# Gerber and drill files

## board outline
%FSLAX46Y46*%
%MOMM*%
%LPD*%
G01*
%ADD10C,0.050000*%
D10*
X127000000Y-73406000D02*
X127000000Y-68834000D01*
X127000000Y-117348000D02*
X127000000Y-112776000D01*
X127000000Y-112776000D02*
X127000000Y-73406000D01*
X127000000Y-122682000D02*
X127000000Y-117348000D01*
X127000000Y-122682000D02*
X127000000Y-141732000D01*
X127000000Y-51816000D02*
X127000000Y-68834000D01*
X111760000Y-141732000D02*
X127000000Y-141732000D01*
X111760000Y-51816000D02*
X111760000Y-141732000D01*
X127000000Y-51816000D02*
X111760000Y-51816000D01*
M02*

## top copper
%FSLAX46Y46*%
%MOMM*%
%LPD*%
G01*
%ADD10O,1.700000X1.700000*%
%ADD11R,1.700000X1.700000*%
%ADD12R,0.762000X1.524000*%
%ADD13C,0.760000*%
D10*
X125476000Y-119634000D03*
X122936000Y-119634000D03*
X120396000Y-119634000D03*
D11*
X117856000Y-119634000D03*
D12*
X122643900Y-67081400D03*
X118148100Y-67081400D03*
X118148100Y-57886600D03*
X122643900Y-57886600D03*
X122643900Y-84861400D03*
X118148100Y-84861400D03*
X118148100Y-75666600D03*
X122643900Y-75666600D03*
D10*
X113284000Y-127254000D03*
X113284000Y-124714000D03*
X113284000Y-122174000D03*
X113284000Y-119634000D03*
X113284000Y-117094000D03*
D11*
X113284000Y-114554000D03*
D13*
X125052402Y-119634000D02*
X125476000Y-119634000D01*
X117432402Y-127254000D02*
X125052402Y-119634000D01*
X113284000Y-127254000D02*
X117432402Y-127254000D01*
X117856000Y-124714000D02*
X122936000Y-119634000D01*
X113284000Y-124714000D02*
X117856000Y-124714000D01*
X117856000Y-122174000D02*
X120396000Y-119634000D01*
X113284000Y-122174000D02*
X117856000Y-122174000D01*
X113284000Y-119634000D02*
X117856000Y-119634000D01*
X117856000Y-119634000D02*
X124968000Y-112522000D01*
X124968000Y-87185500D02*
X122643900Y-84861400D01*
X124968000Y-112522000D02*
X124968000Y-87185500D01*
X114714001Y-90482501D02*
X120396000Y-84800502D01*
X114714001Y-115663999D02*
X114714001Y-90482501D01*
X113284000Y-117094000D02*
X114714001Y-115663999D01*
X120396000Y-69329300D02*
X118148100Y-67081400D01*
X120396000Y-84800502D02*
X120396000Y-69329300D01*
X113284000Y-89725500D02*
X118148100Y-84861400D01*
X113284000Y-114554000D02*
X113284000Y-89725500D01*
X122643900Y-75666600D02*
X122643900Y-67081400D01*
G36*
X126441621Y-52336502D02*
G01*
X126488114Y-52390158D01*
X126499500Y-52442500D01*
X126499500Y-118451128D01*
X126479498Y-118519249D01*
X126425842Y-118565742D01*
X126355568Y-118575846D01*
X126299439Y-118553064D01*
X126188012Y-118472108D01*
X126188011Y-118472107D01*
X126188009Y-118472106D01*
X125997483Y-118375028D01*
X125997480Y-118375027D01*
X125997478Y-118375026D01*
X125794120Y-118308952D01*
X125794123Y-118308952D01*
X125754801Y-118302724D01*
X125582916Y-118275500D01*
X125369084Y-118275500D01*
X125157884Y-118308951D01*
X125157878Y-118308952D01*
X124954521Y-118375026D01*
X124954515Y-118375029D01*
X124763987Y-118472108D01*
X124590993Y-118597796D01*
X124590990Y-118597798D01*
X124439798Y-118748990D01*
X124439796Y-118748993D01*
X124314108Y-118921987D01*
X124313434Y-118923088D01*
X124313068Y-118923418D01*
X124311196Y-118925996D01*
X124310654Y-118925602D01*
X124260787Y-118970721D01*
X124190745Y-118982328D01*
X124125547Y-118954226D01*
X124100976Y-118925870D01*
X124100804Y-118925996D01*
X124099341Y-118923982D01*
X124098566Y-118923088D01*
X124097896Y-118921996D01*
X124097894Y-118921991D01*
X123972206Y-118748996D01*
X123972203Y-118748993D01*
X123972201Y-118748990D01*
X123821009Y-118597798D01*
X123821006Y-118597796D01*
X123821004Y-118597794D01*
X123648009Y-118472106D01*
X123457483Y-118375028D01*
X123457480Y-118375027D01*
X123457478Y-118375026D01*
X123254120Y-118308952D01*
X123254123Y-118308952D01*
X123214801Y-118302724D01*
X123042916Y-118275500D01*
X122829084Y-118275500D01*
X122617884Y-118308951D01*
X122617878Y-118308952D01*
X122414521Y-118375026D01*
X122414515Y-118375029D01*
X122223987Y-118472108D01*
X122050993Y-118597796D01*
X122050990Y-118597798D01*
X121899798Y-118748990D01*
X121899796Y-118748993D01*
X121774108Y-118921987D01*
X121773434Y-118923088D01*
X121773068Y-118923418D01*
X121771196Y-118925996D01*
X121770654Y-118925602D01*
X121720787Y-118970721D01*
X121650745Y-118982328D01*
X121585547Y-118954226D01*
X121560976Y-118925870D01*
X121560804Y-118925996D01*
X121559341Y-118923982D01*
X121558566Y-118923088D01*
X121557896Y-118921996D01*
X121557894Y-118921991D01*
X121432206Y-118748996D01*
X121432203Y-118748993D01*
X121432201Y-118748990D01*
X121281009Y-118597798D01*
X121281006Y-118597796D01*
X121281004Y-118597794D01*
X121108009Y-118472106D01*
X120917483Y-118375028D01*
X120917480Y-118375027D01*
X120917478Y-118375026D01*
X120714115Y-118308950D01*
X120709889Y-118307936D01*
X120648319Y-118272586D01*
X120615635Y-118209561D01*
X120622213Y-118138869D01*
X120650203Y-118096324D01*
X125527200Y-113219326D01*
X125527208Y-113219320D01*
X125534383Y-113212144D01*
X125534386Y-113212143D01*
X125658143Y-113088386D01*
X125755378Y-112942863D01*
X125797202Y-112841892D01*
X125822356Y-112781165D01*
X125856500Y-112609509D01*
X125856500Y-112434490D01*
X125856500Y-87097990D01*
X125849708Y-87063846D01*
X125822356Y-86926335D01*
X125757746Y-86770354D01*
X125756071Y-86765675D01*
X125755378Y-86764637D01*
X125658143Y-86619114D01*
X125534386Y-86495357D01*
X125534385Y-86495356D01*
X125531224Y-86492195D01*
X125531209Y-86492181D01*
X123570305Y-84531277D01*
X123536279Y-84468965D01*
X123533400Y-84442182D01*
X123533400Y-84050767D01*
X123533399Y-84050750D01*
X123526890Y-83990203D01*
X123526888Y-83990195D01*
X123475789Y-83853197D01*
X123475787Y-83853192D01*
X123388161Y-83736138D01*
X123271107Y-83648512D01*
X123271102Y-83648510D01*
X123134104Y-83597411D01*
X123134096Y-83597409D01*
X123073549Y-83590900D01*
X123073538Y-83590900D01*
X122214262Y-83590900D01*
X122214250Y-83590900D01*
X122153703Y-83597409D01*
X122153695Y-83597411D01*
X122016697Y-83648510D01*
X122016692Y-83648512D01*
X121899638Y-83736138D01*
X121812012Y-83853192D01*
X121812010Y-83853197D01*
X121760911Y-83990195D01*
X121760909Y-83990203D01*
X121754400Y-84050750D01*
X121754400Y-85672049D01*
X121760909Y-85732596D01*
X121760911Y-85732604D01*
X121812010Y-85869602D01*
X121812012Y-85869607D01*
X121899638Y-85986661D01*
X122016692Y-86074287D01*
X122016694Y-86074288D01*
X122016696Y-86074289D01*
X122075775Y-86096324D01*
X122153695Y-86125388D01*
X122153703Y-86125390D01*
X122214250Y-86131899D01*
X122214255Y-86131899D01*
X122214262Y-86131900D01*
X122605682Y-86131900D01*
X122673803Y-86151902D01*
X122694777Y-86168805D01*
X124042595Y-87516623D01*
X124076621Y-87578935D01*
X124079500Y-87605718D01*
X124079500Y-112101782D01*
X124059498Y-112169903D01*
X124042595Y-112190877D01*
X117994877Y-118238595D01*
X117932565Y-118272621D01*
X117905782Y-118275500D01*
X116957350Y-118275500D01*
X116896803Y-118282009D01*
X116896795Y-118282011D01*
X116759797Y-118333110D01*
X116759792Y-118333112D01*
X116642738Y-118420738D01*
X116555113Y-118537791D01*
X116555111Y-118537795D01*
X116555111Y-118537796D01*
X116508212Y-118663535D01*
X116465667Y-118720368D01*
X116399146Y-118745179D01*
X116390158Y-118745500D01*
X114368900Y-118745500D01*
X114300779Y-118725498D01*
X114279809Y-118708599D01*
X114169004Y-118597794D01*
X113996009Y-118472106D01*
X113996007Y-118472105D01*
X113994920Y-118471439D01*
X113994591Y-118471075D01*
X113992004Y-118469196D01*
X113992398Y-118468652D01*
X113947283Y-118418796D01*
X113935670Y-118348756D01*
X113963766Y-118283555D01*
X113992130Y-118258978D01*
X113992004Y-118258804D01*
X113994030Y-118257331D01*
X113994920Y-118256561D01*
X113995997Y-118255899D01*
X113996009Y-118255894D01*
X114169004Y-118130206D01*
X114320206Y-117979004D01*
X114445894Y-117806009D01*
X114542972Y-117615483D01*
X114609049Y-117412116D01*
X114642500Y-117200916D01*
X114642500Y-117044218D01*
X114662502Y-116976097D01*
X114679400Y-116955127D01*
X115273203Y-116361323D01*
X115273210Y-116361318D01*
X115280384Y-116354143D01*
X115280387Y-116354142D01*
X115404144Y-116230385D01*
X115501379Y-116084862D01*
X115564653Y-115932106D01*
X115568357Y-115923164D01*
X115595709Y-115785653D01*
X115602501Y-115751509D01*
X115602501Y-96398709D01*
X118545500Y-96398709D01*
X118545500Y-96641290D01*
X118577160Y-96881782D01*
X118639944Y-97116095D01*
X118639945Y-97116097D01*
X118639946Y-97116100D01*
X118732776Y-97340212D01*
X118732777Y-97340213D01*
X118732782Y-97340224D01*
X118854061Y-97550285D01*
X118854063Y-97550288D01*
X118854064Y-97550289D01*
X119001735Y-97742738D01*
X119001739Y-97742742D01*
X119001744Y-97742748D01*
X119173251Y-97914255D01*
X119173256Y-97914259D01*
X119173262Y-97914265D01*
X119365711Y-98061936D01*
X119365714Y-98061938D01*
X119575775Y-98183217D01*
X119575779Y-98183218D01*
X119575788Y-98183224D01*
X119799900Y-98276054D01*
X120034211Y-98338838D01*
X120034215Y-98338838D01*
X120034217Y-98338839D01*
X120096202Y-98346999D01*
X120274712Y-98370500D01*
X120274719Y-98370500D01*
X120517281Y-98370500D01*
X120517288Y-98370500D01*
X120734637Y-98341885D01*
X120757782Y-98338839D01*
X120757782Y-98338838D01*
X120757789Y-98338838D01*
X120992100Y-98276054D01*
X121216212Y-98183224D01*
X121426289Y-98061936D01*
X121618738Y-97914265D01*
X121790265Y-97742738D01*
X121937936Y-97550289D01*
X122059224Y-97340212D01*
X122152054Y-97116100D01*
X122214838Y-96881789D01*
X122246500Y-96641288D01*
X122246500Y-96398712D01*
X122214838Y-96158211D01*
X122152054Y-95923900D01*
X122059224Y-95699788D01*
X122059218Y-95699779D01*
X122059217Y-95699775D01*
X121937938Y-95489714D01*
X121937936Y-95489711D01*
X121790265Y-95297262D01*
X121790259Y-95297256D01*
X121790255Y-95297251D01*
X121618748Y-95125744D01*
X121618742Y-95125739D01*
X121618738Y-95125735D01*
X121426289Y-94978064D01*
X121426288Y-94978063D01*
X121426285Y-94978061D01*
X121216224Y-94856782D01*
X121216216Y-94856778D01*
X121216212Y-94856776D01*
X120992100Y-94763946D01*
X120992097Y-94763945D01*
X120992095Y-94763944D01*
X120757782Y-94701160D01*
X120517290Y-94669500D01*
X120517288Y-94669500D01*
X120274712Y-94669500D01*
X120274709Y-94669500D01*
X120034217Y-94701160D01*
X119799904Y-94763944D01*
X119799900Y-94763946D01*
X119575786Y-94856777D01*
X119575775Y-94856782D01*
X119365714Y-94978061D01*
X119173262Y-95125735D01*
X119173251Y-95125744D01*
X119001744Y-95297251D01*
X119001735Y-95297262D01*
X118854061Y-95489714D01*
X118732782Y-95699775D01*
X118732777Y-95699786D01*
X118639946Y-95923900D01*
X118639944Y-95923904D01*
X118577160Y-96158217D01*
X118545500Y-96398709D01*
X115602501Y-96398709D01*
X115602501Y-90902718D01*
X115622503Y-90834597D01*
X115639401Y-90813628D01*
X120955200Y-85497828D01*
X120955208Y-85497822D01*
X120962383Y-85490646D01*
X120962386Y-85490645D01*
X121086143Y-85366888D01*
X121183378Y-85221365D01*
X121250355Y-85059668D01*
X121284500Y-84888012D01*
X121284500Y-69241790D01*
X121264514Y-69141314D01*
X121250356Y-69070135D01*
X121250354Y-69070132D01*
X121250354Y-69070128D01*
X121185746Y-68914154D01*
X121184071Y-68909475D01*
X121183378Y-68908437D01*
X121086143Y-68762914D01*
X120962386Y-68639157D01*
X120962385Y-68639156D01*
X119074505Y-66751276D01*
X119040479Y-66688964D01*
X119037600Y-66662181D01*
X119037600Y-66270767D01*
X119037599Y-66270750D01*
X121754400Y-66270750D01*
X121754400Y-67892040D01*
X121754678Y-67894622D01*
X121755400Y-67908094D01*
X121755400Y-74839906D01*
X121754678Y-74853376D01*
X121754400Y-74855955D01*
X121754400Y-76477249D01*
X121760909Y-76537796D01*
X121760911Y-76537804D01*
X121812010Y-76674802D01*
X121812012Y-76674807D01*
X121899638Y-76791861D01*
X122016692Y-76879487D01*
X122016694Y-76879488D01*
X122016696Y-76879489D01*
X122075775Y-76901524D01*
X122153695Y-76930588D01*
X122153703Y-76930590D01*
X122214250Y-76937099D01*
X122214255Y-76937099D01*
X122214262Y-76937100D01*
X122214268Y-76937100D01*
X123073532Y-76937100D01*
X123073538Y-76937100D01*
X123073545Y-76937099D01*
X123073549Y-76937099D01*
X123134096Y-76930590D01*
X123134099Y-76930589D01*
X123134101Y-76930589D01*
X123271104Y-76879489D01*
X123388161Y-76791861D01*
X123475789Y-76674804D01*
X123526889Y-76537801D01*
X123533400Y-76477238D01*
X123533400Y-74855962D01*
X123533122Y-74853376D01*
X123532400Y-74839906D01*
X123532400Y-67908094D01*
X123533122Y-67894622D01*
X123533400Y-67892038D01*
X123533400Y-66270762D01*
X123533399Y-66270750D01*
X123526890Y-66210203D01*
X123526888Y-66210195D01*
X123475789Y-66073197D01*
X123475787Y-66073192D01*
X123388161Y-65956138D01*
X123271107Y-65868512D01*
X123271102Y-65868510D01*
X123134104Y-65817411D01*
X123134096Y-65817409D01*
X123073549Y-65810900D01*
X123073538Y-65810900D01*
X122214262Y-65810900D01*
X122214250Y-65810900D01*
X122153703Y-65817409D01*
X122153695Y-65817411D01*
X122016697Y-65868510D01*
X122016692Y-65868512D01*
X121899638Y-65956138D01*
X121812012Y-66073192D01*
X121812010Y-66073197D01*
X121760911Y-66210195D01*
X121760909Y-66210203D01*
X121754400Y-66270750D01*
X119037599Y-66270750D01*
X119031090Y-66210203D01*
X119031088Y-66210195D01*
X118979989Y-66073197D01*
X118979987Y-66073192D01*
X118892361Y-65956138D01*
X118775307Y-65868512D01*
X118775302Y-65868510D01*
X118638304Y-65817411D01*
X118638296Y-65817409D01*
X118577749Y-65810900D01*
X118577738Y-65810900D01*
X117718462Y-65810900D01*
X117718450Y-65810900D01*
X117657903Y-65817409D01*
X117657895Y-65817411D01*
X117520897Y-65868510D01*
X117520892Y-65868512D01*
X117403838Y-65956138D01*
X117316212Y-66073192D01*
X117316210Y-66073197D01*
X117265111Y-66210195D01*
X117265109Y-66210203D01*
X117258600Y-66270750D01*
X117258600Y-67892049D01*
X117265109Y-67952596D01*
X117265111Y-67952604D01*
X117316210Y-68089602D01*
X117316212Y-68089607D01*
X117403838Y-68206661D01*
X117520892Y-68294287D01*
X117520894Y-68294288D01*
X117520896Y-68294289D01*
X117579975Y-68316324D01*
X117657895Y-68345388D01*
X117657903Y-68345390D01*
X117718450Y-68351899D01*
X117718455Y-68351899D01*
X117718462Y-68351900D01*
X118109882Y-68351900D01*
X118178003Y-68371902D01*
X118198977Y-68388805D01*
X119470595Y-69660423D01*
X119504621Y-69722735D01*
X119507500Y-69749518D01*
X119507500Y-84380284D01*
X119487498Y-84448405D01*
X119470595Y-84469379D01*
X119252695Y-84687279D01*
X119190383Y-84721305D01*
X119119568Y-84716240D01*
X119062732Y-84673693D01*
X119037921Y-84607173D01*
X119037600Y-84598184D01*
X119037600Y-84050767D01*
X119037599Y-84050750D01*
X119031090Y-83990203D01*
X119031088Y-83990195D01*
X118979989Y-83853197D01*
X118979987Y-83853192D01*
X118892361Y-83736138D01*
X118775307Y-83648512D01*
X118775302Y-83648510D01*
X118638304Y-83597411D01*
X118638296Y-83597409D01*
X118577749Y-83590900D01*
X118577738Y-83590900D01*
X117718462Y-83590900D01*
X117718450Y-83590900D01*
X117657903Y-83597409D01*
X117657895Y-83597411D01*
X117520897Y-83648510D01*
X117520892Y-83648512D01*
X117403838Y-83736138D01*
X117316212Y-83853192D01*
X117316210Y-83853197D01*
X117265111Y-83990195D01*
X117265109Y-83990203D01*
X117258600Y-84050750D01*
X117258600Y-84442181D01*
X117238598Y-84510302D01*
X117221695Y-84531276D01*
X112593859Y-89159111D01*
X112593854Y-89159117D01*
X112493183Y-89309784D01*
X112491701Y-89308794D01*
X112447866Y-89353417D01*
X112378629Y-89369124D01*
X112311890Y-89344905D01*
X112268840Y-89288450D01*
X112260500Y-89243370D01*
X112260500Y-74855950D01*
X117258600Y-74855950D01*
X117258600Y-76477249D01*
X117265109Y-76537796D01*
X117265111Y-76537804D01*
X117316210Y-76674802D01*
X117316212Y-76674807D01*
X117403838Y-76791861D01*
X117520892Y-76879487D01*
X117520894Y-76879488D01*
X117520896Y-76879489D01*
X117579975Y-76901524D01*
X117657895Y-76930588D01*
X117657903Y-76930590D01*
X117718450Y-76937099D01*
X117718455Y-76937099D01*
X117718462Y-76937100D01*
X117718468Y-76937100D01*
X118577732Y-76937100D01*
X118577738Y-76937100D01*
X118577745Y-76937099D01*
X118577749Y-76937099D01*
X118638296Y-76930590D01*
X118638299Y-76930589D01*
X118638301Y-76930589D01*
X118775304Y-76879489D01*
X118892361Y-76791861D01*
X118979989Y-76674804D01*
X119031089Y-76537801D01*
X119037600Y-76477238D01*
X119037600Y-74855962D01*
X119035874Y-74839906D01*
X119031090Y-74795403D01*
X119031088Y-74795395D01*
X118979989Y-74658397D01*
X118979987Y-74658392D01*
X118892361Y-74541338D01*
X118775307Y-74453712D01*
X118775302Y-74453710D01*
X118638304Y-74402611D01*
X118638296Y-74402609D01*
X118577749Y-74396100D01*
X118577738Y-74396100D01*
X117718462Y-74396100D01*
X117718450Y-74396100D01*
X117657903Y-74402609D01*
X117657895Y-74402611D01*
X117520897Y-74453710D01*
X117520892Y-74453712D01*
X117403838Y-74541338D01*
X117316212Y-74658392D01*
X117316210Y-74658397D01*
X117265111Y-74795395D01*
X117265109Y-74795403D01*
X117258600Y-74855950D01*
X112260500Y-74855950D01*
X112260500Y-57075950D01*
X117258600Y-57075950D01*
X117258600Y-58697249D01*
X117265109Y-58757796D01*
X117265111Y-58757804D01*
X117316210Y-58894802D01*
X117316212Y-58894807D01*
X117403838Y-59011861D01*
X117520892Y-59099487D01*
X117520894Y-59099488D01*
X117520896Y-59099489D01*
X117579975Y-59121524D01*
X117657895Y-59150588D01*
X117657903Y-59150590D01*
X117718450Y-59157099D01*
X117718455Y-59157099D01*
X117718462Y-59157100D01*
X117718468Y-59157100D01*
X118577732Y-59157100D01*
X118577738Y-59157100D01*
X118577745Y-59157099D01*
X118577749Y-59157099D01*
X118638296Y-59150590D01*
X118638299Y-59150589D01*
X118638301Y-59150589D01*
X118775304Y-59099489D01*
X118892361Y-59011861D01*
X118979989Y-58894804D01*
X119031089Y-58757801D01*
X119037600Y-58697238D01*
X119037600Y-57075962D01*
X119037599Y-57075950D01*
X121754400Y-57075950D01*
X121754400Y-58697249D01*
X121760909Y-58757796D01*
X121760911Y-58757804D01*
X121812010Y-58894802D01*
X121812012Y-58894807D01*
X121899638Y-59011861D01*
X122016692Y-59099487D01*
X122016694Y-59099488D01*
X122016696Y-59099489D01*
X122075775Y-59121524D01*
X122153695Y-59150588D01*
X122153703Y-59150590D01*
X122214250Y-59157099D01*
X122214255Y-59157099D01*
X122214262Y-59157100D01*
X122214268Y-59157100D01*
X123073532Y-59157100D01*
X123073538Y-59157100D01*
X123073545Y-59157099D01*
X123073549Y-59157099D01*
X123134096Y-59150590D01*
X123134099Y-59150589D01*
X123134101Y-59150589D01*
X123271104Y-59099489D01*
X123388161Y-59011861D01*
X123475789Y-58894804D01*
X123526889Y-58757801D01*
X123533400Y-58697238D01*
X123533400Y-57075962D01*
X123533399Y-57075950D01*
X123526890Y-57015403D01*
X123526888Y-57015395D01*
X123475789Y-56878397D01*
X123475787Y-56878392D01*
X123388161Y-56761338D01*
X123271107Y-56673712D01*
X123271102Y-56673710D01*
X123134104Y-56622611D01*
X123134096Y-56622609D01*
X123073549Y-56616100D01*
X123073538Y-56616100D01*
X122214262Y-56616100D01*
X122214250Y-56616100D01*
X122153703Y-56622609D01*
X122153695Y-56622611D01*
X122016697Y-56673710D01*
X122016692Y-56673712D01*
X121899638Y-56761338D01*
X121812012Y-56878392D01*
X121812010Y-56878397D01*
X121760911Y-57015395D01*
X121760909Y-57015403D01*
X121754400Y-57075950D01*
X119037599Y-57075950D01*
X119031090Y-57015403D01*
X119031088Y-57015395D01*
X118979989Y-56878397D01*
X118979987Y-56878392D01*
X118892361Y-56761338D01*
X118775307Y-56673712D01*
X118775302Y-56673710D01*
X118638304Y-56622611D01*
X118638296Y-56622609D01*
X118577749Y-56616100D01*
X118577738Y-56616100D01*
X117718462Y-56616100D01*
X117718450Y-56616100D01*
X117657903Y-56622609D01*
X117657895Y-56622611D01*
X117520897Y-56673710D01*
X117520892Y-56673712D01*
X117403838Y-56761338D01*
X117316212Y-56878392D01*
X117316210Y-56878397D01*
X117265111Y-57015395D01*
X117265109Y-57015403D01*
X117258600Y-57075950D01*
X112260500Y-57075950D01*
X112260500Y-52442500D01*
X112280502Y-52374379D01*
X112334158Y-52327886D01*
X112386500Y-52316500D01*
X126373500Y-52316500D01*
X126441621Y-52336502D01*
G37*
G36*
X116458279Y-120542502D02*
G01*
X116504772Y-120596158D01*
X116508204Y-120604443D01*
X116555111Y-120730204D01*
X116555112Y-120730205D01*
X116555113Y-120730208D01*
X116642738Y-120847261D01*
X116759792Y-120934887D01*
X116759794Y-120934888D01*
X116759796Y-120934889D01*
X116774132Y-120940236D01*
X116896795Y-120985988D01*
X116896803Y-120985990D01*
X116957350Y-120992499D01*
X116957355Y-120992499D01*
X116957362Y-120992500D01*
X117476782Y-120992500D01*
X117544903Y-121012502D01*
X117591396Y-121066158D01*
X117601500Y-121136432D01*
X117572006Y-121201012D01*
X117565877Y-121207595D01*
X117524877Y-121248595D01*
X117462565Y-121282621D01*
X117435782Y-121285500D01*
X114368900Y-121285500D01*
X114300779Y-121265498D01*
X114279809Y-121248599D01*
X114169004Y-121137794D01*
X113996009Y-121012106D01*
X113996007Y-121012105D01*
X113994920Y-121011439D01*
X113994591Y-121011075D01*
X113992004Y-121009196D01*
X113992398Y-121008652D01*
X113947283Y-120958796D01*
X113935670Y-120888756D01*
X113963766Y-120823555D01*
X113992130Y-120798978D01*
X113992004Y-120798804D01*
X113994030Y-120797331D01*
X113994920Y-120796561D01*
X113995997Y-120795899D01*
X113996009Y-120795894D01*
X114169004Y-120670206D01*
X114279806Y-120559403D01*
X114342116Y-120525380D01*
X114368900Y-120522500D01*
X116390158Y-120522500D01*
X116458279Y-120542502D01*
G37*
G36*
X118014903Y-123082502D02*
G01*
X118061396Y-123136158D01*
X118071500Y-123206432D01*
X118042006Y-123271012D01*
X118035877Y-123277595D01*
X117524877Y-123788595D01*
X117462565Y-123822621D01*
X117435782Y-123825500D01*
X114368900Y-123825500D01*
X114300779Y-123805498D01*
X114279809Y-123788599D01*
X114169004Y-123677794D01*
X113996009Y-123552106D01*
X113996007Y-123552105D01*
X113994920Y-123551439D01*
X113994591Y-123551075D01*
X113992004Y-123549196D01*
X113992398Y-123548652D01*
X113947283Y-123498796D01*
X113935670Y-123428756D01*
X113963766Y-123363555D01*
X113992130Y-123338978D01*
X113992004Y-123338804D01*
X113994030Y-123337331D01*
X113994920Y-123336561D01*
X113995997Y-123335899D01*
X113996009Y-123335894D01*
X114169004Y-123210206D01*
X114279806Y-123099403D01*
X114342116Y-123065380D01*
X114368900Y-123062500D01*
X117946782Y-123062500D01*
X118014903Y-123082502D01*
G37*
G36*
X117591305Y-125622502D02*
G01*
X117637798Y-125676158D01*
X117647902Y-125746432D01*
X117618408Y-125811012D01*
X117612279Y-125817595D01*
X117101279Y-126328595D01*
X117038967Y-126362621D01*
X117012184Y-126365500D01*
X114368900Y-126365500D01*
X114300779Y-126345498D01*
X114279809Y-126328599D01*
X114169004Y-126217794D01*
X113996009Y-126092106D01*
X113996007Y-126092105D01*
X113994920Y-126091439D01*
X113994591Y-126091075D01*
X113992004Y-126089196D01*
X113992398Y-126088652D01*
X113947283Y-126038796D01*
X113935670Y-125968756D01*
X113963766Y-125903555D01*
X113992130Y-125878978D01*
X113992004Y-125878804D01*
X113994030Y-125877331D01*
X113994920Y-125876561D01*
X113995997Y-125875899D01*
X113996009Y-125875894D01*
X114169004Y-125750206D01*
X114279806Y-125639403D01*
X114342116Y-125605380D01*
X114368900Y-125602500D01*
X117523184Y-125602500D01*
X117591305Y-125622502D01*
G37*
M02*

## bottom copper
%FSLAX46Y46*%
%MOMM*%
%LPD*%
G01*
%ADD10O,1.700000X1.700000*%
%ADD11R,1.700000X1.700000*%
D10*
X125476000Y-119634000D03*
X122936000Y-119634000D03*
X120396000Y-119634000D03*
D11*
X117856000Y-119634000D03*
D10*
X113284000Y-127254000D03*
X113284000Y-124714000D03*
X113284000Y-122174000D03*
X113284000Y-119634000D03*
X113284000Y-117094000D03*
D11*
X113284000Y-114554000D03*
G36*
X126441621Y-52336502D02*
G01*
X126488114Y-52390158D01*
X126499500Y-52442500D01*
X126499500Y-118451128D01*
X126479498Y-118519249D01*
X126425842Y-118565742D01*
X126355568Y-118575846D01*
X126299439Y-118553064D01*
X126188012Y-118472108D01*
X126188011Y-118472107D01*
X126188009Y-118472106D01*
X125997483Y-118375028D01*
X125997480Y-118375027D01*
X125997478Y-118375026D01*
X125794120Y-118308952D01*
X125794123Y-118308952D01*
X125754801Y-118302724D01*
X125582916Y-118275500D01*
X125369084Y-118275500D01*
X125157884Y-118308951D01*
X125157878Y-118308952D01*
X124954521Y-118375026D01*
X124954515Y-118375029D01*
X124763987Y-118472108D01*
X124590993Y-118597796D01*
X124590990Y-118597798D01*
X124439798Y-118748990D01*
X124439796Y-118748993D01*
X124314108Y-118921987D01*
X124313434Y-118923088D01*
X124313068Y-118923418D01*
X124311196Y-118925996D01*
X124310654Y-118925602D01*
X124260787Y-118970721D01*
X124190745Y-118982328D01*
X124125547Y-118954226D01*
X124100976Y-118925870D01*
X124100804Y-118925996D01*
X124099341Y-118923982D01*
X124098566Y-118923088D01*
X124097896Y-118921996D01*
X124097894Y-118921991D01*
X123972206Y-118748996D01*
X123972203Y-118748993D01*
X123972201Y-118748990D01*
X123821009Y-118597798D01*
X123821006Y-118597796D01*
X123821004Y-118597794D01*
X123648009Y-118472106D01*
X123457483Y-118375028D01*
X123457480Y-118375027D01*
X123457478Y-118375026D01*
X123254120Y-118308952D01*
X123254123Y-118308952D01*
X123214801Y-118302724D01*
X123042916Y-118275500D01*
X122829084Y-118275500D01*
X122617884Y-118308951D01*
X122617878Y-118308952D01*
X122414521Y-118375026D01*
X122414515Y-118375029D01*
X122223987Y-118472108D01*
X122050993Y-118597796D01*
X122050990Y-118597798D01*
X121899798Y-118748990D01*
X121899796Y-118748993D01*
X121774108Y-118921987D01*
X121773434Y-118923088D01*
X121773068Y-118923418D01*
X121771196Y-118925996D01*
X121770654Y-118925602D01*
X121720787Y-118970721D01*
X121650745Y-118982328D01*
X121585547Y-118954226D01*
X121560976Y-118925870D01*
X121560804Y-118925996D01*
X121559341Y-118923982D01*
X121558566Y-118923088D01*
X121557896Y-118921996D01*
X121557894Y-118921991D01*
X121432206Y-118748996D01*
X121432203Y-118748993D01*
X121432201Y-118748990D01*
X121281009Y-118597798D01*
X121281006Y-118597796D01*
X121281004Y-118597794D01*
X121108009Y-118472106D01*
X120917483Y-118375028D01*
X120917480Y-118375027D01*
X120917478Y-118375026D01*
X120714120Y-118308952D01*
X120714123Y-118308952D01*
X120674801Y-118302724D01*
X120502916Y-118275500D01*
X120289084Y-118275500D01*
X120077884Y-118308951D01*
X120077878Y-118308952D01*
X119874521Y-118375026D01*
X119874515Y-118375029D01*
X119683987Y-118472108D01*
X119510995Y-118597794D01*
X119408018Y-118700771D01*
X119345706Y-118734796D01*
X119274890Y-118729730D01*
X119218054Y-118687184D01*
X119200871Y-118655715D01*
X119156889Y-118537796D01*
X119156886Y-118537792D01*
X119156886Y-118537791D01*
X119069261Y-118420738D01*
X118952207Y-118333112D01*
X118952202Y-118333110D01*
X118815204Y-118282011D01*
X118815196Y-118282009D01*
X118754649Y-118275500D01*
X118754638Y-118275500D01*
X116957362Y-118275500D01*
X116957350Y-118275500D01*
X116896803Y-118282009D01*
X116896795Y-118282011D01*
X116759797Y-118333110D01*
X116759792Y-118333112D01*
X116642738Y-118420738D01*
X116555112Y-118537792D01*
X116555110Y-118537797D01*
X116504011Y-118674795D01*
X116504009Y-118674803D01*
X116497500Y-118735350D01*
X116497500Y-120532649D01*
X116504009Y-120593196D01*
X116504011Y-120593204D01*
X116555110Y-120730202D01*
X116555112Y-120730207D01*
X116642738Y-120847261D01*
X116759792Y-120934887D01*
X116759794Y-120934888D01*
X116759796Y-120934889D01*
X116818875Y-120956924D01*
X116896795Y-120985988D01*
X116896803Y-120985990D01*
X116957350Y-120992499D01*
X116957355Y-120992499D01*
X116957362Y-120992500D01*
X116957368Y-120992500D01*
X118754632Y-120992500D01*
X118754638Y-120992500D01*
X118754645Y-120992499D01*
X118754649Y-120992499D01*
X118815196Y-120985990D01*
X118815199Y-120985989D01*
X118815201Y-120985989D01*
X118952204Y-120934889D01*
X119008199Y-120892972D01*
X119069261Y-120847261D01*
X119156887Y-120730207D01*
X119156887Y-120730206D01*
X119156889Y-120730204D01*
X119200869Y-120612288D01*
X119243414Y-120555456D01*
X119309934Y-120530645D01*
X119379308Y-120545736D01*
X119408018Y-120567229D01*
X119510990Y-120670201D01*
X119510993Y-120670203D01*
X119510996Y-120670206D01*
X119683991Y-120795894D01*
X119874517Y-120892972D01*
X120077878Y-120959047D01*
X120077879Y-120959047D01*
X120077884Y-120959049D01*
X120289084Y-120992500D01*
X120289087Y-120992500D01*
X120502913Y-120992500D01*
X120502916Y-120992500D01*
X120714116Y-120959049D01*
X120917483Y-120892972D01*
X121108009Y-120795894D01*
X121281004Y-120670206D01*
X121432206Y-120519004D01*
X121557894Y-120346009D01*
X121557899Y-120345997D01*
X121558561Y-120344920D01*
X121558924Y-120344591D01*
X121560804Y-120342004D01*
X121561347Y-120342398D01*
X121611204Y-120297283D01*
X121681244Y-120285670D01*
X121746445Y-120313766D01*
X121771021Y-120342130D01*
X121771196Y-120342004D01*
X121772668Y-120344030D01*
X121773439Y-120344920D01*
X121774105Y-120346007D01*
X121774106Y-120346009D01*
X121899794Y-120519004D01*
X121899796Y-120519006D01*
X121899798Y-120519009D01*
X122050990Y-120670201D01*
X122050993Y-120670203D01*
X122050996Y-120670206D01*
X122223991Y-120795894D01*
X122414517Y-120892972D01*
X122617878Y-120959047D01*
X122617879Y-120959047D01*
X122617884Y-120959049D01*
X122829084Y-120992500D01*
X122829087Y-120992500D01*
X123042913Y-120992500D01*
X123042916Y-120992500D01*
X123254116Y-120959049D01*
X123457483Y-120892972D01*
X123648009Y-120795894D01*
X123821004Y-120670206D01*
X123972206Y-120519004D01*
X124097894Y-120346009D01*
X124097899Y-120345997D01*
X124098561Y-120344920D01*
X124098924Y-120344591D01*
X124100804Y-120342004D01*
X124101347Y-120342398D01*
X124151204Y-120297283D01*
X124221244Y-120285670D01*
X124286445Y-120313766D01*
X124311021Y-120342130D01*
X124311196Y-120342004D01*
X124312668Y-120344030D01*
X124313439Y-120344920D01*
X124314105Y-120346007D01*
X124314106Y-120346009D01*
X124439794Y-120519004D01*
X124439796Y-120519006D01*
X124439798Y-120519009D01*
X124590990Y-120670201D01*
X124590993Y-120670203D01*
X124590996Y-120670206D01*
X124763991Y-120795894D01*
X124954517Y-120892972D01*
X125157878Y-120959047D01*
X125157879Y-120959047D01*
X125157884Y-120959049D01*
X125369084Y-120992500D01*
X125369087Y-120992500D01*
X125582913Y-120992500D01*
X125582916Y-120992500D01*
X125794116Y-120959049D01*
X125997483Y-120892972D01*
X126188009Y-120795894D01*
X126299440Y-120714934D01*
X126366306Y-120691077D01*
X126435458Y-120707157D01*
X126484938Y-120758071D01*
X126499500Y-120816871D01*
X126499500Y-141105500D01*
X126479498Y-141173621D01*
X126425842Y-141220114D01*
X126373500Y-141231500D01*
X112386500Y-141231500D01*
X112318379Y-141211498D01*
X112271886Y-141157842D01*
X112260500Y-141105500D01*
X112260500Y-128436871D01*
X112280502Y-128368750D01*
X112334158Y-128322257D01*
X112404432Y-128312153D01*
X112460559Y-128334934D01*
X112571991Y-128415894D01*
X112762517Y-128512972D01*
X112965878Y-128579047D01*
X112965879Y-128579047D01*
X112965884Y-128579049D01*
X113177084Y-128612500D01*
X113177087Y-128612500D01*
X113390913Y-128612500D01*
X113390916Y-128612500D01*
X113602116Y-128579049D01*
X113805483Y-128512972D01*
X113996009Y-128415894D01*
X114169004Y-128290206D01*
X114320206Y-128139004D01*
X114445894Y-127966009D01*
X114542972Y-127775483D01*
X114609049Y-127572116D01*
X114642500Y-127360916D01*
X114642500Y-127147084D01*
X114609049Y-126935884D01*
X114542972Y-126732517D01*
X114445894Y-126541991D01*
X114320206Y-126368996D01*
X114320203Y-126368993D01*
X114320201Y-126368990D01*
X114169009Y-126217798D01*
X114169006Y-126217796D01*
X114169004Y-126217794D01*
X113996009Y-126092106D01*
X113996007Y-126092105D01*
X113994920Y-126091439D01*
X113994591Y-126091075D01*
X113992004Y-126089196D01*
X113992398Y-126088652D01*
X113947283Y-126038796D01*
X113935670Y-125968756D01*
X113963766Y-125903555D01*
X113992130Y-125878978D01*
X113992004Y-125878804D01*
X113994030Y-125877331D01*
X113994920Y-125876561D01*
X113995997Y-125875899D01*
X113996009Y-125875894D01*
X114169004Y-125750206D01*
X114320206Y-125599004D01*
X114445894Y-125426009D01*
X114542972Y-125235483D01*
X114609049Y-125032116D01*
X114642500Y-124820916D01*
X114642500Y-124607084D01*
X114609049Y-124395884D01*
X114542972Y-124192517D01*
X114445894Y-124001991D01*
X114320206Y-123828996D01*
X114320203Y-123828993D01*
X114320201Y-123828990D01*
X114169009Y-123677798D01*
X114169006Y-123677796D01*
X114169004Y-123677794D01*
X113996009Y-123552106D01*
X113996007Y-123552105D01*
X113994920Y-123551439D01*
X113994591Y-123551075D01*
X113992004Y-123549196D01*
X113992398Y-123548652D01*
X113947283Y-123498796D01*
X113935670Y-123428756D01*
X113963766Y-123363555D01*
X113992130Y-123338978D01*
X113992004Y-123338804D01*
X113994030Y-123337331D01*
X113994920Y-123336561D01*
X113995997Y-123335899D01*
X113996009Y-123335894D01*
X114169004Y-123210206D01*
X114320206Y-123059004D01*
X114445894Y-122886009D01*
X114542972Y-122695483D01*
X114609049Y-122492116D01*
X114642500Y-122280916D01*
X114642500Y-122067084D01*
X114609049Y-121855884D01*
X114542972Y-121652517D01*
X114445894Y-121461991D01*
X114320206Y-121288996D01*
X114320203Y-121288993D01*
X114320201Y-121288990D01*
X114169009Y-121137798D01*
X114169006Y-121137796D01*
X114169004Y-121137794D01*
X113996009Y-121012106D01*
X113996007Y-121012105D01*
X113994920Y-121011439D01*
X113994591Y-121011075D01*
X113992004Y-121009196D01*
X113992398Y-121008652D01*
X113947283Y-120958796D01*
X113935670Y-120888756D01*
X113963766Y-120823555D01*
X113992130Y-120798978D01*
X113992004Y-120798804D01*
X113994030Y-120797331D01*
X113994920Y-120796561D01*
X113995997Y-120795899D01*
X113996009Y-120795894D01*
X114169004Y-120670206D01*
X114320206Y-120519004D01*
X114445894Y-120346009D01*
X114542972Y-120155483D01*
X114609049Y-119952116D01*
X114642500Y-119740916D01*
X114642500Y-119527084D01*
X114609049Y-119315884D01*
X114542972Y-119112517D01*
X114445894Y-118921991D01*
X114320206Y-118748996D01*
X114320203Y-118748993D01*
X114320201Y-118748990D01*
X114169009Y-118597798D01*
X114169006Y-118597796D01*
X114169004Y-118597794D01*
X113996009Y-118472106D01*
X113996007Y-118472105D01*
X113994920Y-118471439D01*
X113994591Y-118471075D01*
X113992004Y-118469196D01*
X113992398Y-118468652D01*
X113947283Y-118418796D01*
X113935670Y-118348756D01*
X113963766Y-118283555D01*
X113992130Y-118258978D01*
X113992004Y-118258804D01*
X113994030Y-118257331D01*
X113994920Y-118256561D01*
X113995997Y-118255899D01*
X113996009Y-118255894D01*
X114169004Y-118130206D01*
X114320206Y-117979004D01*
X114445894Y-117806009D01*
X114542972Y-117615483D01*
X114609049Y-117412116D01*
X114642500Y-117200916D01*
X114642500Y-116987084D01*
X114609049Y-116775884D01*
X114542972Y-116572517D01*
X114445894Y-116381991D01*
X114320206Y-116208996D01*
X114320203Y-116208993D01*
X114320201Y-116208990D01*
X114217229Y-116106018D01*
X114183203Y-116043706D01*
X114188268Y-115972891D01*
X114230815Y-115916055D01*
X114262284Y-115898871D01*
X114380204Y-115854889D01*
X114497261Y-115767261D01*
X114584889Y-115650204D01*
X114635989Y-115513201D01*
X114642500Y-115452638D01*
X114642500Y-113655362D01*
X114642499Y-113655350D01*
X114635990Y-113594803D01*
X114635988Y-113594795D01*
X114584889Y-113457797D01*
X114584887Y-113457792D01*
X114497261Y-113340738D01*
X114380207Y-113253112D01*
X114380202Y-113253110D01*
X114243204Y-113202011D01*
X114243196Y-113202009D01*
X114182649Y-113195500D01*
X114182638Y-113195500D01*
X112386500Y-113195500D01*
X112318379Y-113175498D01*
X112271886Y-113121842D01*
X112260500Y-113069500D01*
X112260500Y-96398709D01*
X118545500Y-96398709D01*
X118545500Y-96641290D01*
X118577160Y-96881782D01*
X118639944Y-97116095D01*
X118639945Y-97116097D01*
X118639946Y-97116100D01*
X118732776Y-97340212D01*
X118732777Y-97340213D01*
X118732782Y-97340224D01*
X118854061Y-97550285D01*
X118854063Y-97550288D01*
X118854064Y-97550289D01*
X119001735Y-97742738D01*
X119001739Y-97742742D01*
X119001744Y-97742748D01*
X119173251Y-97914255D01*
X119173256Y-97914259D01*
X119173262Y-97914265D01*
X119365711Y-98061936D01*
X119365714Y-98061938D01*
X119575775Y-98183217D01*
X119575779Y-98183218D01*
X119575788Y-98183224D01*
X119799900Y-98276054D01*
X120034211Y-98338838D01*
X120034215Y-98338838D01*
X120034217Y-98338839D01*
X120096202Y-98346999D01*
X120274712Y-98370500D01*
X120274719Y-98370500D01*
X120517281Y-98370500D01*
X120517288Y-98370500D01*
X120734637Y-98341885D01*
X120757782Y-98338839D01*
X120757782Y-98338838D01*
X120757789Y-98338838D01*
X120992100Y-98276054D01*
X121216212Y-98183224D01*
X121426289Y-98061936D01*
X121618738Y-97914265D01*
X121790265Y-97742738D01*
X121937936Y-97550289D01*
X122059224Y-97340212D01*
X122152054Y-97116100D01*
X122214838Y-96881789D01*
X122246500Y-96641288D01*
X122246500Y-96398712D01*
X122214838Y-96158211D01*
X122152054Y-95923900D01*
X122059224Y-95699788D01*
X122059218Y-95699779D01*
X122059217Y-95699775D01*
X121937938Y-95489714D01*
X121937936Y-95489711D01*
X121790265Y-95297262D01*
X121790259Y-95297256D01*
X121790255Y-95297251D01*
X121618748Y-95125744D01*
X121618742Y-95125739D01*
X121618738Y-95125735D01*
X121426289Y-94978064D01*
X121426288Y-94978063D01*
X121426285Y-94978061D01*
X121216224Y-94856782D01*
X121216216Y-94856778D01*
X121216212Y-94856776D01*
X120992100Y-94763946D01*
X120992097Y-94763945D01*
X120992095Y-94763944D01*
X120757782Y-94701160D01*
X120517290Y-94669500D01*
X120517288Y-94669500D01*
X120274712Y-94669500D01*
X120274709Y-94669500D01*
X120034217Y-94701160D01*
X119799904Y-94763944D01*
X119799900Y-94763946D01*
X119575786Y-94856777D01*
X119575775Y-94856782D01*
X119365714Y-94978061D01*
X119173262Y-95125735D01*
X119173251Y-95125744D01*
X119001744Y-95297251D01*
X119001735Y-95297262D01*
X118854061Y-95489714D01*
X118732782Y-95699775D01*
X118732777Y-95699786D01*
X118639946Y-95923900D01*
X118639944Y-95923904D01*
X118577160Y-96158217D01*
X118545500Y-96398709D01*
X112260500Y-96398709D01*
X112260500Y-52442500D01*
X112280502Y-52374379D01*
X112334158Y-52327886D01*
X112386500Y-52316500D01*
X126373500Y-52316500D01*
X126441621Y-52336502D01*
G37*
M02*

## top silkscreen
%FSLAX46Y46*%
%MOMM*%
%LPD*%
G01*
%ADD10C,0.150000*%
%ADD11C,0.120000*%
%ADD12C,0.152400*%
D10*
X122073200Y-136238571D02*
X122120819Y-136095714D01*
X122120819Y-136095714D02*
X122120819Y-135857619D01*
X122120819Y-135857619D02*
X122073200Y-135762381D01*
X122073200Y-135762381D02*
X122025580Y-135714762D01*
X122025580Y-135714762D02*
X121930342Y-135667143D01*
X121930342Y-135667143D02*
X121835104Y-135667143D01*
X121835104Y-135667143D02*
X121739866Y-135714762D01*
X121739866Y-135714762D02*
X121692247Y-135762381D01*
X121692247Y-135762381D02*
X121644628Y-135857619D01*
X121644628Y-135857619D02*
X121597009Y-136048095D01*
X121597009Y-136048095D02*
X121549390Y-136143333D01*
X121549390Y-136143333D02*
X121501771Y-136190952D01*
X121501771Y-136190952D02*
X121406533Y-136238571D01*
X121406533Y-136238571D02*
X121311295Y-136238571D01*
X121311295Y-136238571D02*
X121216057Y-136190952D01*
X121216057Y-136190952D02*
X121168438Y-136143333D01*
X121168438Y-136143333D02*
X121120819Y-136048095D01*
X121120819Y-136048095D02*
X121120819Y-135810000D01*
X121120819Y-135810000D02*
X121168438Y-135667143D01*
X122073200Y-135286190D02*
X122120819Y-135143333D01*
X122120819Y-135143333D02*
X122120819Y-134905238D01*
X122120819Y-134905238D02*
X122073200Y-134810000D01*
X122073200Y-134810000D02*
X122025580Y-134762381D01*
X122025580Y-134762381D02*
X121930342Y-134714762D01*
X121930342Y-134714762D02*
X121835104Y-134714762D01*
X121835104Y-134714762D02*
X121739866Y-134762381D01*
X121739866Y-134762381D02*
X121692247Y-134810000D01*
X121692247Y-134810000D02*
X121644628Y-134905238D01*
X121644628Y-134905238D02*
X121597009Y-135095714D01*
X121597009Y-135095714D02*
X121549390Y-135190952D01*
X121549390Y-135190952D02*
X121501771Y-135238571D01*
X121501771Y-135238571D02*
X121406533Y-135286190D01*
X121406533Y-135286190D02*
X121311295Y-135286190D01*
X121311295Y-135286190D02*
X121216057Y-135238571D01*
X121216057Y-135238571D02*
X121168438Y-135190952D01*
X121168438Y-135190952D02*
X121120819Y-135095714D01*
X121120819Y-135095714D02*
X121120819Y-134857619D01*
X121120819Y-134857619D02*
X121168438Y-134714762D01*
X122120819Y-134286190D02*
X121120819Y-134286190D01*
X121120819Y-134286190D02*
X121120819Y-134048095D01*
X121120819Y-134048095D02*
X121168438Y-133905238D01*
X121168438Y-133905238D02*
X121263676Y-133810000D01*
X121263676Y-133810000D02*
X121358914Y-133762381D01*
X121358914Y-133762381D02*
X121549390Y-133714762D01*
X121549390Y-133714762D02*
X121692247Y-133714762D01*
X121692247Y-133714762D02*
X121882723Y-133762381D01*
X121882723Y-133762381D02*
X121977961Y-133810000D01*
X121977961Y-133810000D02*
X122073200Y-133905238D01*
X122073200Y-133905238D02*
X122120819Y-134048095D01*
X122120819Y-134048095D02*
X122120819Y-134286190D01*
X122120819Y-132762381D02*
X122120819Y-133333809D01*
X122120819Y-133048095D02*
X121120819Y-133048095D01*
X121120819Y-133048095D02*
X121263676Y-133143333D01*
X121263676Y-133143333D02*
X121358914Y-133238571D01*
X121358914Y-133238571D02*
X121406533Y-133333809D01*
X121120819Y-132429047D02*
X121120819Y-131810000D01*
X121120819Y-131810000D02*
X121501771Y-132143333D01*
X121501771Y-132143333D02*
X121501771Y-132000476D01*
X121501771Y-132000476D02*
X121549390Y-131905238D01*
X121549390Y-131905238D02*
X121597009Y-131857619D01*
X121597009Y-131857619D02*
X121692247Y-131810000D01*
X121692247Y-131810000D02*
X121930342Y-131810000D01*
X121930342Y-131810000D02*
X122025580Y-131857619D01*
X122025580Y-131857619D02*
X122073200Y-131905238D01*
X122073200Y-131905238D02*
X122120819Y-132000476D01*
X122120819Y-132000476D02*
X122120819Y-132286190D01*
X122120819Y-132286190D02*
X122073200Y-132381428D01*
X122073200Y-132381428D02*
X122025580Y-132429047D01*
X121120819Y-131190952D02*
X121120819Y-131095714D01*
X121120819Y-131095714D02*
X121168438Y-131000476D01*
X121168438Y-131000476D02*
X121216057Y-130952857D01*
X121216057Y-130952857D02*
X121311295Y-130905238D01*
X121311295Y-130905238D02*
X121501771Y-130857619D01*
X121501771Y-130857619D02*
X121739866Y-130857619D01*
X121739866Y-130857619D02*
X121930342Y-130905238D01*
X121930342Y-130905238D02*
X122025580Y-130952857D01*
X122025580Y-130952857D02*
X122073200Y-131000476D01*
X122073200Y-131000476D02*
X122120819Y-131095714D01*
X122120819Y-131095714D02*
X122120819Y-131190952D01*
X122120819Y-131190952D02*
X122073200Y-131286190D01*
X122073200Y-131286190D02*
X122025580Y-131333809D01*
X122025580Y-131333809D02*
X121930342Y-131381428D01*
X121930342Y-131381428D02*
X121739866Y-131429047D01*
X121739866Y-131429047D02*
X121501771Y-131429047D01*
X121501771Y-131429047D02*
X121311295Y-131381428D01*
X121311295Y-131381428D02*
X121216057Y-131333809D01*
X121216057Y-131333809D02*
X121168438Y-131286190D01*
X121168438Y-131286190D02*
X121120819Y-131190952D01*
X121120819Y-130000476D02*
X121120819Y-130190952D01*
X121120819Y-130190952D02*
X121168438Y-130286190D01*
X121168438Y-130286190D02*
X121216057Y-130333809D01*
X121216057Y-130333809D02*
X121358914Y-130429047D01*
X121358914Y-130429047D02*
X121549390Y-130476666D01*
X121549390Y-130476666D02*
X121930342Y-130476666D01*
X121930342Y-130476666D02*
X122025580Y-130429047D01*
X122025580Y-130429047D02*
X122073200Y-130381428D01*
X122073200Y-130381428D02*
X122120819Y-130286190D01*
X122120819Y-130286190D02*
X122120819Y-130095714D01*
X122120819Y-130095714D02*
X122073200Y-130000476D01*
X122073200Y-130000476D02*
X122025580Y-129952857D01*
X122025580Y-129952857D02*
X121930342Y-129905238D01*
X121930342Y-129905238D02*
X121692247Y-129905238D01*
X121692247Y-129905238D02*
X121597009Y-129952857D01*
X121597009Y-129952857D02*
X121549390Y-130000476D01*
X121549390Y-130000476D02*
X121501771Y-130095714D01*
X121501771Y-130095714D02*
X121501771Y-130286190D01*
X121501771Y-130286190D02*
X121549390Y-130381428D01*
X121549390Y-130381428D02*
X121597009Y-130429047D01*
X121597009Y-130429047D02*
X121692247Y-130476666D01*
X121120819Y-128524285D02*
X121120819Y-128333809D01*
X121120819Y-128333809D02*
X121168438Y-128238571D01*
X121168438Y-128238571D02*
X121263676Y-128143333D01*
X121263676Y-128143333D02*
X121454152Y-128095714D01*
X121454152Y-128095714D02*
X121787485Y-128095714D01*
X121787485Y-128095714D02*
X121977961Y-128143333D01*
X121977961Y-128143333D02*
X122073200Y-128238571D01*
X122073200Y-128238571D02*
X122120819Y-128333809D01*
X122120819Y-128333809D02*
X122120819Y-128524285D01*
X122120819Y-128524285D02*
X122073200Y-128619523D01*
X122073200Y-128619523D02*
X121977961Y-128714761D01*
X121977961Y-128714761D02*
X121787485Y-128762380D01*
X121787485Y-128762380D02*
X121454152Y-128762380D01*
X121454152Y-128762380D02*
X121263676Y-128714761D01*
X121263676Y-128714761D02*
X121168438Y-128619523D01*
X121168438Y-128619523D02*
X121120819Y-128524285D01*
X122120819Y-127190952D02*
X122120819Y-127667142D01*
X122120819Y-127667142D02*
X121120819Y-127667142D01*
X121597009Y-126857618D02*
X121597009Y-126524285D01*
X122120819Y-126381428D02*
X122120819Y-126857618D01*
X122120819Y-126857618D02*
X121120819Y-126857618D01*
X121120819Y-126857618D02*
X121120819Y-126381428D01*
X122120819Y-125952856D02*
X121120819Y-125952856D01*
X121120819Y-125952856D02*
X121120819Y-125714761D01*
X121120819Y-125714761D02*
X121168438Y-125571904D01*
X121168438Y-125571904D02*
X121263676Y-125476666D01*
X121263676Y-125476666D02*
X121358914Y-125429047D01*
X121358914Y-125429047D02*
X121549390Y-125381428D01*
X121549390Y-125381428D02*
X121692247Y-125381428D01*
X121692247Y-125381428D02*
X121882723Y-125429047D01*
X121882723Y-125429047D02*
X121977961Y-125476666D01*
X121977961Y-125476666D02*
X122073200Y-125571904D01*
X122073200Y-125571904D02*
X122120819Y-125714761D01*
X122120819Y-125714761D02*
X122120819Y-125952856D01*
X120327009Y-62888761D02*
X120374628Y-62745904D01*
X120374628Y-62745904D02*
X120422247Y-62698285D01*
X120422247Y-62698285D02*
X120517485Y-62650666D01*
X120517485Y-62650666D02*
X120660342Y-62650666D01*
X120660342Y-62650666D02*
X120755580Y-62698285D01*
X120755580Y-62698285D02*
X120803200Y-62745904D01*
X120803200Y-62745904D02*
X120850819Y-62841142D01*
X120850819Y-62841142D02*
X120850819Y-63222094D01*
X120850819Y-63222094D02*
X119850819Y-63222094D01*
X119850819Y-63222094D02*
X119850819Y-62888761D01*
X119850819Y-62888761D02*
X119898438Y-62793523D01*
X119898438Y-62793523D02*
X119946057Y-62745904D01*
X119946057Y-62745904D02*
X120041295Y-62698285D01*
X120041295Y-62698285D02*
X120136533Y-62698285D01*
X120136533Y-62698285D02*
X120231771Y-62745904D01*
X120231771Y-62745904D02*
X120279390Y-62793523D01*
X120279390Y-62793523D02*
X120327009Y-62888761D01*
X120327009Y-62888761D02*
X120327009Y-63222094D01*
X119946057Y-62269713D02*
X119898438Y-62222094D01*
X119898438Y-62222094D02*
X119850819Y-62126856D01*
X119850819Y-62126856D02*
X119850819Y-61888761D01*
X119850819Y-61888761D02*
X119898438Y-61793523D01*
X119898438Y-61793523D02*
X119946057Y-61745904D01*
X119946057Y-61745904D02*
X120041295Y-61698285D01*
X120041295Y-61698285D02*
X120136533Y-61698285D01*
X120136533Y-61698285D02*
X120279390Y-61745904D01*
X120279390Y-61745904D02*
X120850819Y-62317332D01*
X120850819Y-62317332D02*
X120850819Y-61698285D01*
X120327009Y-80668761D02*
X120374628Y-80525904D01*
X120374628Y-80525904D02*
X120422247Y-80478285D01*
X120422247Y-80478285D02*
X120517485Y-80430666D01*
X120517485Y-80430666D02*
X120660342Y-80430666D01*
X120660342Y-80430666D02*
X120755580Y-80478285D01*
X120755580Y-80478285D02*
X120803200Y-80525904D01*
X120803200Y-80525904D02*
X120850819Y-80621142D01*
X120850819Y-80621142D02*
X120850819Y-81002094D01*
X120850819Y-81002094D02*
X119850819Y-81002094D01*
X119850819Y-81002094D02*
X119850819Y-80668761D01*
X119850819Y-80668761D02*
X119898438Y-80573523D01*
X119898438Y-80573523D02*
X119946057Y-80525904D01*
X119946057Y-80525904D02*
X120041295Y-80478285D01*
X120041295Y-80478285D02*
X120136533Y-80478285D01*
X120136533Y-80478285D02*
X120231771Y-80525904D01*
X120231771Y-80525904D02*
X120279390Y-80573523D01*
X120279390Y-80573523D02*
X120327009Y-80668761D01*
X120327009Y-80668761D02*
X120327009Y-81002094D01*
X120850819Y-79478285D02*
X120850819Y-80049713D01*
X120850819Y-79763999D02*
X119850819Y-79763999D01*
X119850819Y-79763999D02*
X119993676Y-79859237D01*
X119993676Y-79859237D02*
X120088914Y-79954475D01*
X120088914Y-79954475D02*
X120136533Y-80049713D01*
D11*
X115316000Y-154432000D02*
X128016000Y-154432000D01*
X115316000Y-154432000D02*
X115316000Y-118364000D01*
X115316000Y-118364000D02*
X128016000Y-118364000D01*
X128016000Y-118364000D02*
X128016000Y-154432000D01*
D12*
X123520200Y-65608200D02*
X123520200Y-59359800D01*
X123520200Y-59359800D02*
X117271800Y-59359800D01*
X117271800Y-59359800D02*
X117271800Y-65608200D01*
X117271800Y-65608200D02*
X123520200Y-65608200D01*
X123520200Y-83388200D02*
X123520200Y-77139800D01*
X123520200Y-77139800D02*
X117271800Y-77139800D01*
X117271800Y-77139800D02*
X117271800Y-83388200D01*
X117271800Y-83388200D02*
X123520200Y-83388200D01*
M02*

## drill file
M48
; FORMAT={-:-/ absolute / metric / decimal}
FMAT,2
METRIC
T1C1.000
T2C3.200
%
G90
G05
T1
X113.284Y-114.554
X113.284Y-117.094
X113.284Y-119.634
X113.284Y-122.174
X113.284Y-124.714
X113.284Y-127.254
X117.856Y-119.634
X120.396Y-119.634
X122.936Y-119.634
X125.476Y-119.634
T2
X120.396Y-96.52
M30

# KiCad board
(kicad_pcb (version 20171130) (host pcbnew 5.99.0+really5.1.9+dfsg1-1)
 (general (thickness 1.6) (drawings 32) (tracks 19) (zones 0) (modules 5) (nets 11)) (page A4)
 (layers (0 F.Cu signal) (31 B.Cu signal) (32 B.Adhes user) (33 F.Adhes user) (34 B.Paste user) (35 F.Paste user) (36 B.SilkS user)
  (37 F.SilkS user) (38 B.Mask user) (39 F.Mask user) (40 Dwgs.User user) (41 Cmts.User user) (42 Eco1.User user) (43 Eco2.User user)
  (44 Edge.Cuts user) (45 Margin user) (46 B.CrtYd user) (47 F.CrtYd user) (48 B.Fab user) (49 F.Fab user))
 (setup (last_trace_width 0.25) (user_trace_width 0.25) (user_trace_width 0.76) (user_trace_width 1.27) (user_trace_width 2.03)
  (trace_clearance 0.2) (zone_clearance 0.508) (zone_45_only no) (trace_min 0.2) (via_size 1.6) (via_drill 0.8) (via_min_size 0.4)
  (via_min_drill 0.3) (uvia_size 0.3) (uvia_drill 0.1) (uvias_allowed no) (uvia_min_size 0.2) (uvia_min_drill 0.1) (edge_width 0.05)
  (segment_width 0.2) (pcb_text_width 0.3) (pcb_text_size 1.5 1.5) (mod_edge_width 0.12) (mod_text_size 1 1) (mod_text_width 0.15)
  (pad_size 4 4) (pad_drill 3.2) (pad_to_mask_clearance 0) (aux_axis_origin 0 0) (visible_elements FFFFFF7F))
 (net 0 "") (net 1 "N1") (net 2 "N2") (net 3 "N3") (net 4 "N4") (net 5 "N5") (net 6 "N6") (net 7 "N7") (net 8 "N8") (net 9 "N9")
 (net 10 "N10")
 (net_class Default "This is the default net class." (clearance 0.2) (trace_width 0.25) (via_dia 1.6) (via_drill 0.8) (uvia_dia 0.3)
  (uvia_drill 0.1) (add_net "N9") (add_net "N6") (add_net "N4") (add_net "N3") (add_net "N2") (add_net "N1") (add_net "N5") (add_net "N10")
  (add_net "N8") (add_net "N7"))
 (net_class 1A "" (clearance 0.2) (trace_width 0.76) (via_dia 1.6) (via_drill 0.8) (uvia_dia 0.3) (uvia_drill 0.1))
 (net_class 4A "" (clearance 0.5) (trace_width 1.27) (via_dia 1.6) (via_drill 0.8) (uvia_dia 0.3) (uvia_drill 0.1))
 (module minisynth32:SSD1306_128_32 (layer F.Cu) (at 121.666 136.398 90)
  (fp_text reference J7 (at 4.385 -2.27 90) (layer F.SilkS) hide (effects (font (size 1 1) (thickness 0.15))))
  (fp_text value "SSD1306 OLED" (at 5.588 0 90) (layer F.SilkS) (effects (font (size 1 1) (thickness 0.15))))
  (fp_line (start -18.034 -6.35) (end -18.034 6.35) (layer F.SilkS) (width 0.12))
  (fp_line (start -18.034 -6.35) (end 18.034 -6.35) (layer F.SilkS) (width 0.12))
  (fp_line (start 18.034 -6.35) (end 18.034 6.35) (layer F.SilkS) (width 0.12))
  (fp_line (start 18.034 6.35) (end -18.034 6.35) (layer F.SilkS) (width 0.12))
  (pad 4 thru_hole oval (at 16.764 3.81 90) (size 1.7 1.7) (drill 1) (layers *.Cu *.Mask) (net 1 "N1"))
  (pad 3 thru_hole oval (at 16.764 1.27 90) (size 1.7 1.7) (drill 1) (layers *.Cu *.Mask) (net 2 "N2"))
  (pad 2 thru_hole oval (at 16.764 -1.27 90) (size 1.7 1.7) (drill 1) (layers *.Cu *.Mask) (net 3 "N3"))
  (pad 1 thru_hole rect (at 16.764 -3.81 90) (size 1.7 1.7) (drill 1) (layers *.Cu *.Mask) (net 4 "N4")))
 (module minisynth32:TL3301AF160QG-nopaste (layer F.Cu) (at 120.396 62.484 90)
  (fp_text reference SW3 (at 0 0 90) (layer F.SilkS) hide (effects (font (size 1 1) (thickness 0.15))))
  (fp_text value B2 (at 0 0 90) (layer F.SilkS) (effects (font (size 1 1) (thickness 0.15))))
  (fp_line (start -3.1242 3.1242) (end 3.1242 3.1242) (layer F.SilkS) (width 0.1524))
  (fp_line (start 3.1242 3.1242) (end 3.1242 -3.1242) (layer F.SilkS) (width 0.1524))
  (fp_line (start 3.1242 -3.1242) (end -3.1242 -3.1242) (layer F.SilkS) (width 0.1524))
  (fp_line (start -3.1242 -3.1242) (end -3.1242 3.1242) (layer F.SilkS) (width 0.1524))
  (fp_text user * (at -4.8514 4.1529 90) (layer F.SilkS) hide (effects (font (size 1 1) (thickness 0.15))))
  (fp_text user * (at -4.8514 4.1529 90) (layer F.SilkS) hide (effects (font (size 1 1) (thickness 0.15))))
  (pad 1 smd rect (at -4.5974 2.2479 90) (size 1.524 0.762) (layers F.Cu F.Mask) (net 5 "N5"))
  (pad 3 smd rect (at -4.5974 -2.2479 90) (size 1.524 0.762) (layers F.Cu F.Mask) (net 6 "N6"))
  (pad 4 smd rect (at 4.5974 -2.2479 90) (size 1.524 0.762) (layers F.Cu F.Mask) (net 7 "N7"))
  (pad 2 smd rect (at 4.5974 2.2479 90) (size 1.524 0.762) (layers F.Cu F.Mask) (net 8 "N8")))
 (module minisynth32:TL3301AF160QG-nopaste (layer F.Cu) (at 120.396 80.264 90)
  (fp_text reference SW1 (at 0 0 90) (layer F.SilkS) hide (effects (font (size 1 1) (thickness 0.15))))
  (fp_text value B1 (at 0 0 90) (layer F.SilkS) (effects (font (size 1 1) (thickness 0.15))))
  (fp_line (start -3.1242 3.1242) (end 3.1242 3.1242) (layer F.SilkS) (width 0.1524))
  (fp_line (start 3.1242 3.1242) (end 3.1242 -3.1242) (layer F.SilkS) (width 0.1524))
  (fp_line (start 3.1242 -3.1242) (end -3.1242 -3.1242) (layer F.SilkS) (width 0.1524))
  (fp_line (start -3.1242 -3.1242) (end -3.1242 3.1242) (layer F.SilkS) (width 0.1524))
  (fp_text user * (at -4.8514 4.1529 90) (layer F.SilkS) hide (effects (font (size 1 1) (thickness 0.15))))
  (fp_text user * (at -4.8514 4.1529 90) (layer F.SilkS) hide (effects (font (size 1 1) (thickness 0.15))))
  (pad 1 smd rect (at -4.5974 2.2479 90) (size 1.524 0.762) (layers F.Cu F.Mask) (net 4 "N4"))
  (pad 3 smd rect (at -4.5974 -2.2479 90) (size 1.524 0.762) (layers F.Cu F.Mask) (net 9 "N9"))
  (pad 4 smd rect (at 4.5974 -2.2479 90) (size 1.524 0.762) (layers F.Cu F.Mask) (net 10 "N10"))
  (pad 2 smd rect (at 4.5974 2.2479 90) (size 1.524 0.762) (layers F.Cu F.Mask) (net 5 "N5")))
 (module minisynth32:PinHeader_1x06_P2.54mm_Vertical (layer B.Cu) (at 113.284 114.554 180)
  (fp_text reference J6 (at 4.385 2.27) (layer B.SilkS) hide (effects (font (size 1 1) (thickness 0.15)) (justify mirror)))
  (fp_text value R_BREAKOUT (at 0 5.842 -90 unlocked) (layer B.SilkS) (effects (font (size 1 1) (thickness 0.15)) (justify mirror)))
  (pad 6 thru_hole oval (at 0 -12.7 180) (size 1.7 1.7) (drill 1) (layers *.Cu *.Mask) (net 1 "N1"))
  (pad 5 thru_hole oval (at 0 -10.16 180) (size 1.7 1.7) (drill 1) (layers *.Cu *.Mask) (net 2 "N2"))
  (pad 4 thru_hole oval (at 0 -7.62 180) (size 1.7 1.7) (drill 1) (layers *.Cu *.Mask) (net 3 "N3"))
  (pad 3 thru_hole oval (at 0 -5.08 180) (size 1.7 1.7) (drill 1) (layers *.Cu *.Mask) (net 4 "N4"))
  (pad 2 thru_hole oval (at 0 -2.54 180) (size 1.7 1.7) (drill 1) (layers *.Cu *.Mask) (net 6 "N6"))
  (pad 1 thru_hole rect (at 0 0 180) (size 1.7 1.7) (drill 1) (layers *.Cu *.Mask) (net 9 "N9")))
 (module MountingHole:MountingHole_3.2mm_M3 (layer F.Cu) (at 120.396 96.52)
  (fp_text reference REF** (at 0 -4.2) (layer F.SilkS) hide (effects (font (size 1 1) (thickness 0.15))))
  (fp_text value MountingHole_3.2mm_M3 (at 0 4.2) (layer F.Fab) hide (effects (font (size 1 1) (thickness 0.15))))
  (pad 1 np_thru_hole circle (at 0 0) (size 3.2 3.2) (drill 3.2) (layers *.Cu *.Mask)))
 (gr_line (start 127 73.406) (end 127 68.834) (layer Edge.Cuts) (width 0.05))
 (gr_line (start 127 117.348) (end 127 112.776) (layer Edge.Cuts) (width 0.05))
 (gr_line (start 127 112.776) (end 127 73.406) (layer Edge.Cuts) (width 0.05))
 (gr_line (start 127 122.682) (end 127 117.348) (layer Edge.Cuts) (width 0.05))
 (gr_line (start 127 122.682) (end 127 141.732) (layer Edge.Cuts) (width 0.05))
 (gr_line (start 127 51.816) (end 127 68.834) (layer Edge.Cuts) (width 0.05))
 (gr_line (start 111.76 141.732) (end 127 141.732) (layer Edge.Cuts) (width 0.05))
 (gr_line (start 111.76 51.816) (end 111.76 141.732) (layer Edge.Cuts) (width 0.05))
 (gr_line (start 127 51.816) (end 111.76 51.816) (layer Edge.Cuts) (width 0.05))
 (segment (start 125.052402 119.634) (end 125.476 119.634) (width 0.76) (layer F.Cu) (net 1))
 (segment (start 117.432402 127.254) (end 125.052402 119.634) (width 0.76) (layer F.Cu) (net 1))
 (segment (start 113.284 127.254) (end 117.432402 127.254) (width 0.76) (layer F.Cu) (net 1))
 (segment (start 117.856 124.714) (end 122.936 119.634) (width 0.76) (layer F.Cu) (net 2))
 (segment (start 113.284 124.714) (end 117.856 124.714) (width 0.76) (layer F.Cu) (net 2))
 (segment (start 117.856 122.174) (end 120.396 119.634) (width 0.76) (layer F.Cu) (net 3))
 (segment (start 113.284 122.174) (end 117.856 122.174) (width 0.76) (layer F.Cu) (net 3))
 (segment (start 113.284 119.634) (end 117.856 119.634) (width 0.76) (layer F.Cu) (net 4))
 (segment (start 117.856 119.634) (end 124.968 112.522) (width 0.76) (layer F.Cu) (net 4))
 (segment (start 124.968 87.1855) (end 122.6439 84.8614) (width 0.76) (layer F.Cu) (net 4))
 (segment (start 124.968 112.522) (end 124.968 87.1855) (width 0.76) (layer F.Cu) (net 4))
 (segment (start 114.714001 90.482501) (end 120.396 84.800502) (width 0.76) (layer F.Cu) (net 6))
 (segment (start 114.714001 115.663999) (end 114.714001 90.482501) (width 0.76) (layer F.Cu) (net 6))
 (segment (start 113.284 117.094) (end 114.714001 115.663999) (width 0.76) (layer F.Cu) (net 6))
 (segment (start 120.396 69.3293) (end 118.1481 67.0814) (width 0.76) (layer F.Cu) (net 6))
 (segment (start 120.396 84.800502) (end 120.396 69.3293) (width 0.76) (layer F.Cu) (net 6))
 (segment (start 113.284 89.7255) (end 118.1481 84.8614) (width 0.76) (layer F.Cu) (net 9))
 (segment (start 113.284 114.554) (end 113.284 89.7255) (width 0.76) (layer F.Cu) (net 9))
 (segment (start 122.6439 75.6666) (end 122.6439 67.0814) (width 0.76) (layer F.Cu) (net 5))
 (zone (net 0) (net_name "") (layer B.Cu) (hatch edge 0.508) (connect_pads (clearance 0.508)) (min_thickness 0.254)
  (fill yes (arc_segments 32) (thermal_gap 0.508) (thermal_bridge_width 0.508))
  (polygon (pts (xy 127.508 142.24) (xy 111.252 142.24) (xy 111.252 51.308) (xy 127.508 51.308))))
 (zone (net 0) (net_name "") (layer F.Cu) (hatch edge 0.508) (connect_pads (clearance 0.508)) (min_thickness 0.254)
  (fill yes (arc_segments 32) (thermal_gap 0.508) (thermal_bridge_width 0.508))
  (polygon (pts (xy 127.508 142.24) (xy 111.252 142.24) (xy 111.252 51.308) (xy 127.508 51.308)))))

